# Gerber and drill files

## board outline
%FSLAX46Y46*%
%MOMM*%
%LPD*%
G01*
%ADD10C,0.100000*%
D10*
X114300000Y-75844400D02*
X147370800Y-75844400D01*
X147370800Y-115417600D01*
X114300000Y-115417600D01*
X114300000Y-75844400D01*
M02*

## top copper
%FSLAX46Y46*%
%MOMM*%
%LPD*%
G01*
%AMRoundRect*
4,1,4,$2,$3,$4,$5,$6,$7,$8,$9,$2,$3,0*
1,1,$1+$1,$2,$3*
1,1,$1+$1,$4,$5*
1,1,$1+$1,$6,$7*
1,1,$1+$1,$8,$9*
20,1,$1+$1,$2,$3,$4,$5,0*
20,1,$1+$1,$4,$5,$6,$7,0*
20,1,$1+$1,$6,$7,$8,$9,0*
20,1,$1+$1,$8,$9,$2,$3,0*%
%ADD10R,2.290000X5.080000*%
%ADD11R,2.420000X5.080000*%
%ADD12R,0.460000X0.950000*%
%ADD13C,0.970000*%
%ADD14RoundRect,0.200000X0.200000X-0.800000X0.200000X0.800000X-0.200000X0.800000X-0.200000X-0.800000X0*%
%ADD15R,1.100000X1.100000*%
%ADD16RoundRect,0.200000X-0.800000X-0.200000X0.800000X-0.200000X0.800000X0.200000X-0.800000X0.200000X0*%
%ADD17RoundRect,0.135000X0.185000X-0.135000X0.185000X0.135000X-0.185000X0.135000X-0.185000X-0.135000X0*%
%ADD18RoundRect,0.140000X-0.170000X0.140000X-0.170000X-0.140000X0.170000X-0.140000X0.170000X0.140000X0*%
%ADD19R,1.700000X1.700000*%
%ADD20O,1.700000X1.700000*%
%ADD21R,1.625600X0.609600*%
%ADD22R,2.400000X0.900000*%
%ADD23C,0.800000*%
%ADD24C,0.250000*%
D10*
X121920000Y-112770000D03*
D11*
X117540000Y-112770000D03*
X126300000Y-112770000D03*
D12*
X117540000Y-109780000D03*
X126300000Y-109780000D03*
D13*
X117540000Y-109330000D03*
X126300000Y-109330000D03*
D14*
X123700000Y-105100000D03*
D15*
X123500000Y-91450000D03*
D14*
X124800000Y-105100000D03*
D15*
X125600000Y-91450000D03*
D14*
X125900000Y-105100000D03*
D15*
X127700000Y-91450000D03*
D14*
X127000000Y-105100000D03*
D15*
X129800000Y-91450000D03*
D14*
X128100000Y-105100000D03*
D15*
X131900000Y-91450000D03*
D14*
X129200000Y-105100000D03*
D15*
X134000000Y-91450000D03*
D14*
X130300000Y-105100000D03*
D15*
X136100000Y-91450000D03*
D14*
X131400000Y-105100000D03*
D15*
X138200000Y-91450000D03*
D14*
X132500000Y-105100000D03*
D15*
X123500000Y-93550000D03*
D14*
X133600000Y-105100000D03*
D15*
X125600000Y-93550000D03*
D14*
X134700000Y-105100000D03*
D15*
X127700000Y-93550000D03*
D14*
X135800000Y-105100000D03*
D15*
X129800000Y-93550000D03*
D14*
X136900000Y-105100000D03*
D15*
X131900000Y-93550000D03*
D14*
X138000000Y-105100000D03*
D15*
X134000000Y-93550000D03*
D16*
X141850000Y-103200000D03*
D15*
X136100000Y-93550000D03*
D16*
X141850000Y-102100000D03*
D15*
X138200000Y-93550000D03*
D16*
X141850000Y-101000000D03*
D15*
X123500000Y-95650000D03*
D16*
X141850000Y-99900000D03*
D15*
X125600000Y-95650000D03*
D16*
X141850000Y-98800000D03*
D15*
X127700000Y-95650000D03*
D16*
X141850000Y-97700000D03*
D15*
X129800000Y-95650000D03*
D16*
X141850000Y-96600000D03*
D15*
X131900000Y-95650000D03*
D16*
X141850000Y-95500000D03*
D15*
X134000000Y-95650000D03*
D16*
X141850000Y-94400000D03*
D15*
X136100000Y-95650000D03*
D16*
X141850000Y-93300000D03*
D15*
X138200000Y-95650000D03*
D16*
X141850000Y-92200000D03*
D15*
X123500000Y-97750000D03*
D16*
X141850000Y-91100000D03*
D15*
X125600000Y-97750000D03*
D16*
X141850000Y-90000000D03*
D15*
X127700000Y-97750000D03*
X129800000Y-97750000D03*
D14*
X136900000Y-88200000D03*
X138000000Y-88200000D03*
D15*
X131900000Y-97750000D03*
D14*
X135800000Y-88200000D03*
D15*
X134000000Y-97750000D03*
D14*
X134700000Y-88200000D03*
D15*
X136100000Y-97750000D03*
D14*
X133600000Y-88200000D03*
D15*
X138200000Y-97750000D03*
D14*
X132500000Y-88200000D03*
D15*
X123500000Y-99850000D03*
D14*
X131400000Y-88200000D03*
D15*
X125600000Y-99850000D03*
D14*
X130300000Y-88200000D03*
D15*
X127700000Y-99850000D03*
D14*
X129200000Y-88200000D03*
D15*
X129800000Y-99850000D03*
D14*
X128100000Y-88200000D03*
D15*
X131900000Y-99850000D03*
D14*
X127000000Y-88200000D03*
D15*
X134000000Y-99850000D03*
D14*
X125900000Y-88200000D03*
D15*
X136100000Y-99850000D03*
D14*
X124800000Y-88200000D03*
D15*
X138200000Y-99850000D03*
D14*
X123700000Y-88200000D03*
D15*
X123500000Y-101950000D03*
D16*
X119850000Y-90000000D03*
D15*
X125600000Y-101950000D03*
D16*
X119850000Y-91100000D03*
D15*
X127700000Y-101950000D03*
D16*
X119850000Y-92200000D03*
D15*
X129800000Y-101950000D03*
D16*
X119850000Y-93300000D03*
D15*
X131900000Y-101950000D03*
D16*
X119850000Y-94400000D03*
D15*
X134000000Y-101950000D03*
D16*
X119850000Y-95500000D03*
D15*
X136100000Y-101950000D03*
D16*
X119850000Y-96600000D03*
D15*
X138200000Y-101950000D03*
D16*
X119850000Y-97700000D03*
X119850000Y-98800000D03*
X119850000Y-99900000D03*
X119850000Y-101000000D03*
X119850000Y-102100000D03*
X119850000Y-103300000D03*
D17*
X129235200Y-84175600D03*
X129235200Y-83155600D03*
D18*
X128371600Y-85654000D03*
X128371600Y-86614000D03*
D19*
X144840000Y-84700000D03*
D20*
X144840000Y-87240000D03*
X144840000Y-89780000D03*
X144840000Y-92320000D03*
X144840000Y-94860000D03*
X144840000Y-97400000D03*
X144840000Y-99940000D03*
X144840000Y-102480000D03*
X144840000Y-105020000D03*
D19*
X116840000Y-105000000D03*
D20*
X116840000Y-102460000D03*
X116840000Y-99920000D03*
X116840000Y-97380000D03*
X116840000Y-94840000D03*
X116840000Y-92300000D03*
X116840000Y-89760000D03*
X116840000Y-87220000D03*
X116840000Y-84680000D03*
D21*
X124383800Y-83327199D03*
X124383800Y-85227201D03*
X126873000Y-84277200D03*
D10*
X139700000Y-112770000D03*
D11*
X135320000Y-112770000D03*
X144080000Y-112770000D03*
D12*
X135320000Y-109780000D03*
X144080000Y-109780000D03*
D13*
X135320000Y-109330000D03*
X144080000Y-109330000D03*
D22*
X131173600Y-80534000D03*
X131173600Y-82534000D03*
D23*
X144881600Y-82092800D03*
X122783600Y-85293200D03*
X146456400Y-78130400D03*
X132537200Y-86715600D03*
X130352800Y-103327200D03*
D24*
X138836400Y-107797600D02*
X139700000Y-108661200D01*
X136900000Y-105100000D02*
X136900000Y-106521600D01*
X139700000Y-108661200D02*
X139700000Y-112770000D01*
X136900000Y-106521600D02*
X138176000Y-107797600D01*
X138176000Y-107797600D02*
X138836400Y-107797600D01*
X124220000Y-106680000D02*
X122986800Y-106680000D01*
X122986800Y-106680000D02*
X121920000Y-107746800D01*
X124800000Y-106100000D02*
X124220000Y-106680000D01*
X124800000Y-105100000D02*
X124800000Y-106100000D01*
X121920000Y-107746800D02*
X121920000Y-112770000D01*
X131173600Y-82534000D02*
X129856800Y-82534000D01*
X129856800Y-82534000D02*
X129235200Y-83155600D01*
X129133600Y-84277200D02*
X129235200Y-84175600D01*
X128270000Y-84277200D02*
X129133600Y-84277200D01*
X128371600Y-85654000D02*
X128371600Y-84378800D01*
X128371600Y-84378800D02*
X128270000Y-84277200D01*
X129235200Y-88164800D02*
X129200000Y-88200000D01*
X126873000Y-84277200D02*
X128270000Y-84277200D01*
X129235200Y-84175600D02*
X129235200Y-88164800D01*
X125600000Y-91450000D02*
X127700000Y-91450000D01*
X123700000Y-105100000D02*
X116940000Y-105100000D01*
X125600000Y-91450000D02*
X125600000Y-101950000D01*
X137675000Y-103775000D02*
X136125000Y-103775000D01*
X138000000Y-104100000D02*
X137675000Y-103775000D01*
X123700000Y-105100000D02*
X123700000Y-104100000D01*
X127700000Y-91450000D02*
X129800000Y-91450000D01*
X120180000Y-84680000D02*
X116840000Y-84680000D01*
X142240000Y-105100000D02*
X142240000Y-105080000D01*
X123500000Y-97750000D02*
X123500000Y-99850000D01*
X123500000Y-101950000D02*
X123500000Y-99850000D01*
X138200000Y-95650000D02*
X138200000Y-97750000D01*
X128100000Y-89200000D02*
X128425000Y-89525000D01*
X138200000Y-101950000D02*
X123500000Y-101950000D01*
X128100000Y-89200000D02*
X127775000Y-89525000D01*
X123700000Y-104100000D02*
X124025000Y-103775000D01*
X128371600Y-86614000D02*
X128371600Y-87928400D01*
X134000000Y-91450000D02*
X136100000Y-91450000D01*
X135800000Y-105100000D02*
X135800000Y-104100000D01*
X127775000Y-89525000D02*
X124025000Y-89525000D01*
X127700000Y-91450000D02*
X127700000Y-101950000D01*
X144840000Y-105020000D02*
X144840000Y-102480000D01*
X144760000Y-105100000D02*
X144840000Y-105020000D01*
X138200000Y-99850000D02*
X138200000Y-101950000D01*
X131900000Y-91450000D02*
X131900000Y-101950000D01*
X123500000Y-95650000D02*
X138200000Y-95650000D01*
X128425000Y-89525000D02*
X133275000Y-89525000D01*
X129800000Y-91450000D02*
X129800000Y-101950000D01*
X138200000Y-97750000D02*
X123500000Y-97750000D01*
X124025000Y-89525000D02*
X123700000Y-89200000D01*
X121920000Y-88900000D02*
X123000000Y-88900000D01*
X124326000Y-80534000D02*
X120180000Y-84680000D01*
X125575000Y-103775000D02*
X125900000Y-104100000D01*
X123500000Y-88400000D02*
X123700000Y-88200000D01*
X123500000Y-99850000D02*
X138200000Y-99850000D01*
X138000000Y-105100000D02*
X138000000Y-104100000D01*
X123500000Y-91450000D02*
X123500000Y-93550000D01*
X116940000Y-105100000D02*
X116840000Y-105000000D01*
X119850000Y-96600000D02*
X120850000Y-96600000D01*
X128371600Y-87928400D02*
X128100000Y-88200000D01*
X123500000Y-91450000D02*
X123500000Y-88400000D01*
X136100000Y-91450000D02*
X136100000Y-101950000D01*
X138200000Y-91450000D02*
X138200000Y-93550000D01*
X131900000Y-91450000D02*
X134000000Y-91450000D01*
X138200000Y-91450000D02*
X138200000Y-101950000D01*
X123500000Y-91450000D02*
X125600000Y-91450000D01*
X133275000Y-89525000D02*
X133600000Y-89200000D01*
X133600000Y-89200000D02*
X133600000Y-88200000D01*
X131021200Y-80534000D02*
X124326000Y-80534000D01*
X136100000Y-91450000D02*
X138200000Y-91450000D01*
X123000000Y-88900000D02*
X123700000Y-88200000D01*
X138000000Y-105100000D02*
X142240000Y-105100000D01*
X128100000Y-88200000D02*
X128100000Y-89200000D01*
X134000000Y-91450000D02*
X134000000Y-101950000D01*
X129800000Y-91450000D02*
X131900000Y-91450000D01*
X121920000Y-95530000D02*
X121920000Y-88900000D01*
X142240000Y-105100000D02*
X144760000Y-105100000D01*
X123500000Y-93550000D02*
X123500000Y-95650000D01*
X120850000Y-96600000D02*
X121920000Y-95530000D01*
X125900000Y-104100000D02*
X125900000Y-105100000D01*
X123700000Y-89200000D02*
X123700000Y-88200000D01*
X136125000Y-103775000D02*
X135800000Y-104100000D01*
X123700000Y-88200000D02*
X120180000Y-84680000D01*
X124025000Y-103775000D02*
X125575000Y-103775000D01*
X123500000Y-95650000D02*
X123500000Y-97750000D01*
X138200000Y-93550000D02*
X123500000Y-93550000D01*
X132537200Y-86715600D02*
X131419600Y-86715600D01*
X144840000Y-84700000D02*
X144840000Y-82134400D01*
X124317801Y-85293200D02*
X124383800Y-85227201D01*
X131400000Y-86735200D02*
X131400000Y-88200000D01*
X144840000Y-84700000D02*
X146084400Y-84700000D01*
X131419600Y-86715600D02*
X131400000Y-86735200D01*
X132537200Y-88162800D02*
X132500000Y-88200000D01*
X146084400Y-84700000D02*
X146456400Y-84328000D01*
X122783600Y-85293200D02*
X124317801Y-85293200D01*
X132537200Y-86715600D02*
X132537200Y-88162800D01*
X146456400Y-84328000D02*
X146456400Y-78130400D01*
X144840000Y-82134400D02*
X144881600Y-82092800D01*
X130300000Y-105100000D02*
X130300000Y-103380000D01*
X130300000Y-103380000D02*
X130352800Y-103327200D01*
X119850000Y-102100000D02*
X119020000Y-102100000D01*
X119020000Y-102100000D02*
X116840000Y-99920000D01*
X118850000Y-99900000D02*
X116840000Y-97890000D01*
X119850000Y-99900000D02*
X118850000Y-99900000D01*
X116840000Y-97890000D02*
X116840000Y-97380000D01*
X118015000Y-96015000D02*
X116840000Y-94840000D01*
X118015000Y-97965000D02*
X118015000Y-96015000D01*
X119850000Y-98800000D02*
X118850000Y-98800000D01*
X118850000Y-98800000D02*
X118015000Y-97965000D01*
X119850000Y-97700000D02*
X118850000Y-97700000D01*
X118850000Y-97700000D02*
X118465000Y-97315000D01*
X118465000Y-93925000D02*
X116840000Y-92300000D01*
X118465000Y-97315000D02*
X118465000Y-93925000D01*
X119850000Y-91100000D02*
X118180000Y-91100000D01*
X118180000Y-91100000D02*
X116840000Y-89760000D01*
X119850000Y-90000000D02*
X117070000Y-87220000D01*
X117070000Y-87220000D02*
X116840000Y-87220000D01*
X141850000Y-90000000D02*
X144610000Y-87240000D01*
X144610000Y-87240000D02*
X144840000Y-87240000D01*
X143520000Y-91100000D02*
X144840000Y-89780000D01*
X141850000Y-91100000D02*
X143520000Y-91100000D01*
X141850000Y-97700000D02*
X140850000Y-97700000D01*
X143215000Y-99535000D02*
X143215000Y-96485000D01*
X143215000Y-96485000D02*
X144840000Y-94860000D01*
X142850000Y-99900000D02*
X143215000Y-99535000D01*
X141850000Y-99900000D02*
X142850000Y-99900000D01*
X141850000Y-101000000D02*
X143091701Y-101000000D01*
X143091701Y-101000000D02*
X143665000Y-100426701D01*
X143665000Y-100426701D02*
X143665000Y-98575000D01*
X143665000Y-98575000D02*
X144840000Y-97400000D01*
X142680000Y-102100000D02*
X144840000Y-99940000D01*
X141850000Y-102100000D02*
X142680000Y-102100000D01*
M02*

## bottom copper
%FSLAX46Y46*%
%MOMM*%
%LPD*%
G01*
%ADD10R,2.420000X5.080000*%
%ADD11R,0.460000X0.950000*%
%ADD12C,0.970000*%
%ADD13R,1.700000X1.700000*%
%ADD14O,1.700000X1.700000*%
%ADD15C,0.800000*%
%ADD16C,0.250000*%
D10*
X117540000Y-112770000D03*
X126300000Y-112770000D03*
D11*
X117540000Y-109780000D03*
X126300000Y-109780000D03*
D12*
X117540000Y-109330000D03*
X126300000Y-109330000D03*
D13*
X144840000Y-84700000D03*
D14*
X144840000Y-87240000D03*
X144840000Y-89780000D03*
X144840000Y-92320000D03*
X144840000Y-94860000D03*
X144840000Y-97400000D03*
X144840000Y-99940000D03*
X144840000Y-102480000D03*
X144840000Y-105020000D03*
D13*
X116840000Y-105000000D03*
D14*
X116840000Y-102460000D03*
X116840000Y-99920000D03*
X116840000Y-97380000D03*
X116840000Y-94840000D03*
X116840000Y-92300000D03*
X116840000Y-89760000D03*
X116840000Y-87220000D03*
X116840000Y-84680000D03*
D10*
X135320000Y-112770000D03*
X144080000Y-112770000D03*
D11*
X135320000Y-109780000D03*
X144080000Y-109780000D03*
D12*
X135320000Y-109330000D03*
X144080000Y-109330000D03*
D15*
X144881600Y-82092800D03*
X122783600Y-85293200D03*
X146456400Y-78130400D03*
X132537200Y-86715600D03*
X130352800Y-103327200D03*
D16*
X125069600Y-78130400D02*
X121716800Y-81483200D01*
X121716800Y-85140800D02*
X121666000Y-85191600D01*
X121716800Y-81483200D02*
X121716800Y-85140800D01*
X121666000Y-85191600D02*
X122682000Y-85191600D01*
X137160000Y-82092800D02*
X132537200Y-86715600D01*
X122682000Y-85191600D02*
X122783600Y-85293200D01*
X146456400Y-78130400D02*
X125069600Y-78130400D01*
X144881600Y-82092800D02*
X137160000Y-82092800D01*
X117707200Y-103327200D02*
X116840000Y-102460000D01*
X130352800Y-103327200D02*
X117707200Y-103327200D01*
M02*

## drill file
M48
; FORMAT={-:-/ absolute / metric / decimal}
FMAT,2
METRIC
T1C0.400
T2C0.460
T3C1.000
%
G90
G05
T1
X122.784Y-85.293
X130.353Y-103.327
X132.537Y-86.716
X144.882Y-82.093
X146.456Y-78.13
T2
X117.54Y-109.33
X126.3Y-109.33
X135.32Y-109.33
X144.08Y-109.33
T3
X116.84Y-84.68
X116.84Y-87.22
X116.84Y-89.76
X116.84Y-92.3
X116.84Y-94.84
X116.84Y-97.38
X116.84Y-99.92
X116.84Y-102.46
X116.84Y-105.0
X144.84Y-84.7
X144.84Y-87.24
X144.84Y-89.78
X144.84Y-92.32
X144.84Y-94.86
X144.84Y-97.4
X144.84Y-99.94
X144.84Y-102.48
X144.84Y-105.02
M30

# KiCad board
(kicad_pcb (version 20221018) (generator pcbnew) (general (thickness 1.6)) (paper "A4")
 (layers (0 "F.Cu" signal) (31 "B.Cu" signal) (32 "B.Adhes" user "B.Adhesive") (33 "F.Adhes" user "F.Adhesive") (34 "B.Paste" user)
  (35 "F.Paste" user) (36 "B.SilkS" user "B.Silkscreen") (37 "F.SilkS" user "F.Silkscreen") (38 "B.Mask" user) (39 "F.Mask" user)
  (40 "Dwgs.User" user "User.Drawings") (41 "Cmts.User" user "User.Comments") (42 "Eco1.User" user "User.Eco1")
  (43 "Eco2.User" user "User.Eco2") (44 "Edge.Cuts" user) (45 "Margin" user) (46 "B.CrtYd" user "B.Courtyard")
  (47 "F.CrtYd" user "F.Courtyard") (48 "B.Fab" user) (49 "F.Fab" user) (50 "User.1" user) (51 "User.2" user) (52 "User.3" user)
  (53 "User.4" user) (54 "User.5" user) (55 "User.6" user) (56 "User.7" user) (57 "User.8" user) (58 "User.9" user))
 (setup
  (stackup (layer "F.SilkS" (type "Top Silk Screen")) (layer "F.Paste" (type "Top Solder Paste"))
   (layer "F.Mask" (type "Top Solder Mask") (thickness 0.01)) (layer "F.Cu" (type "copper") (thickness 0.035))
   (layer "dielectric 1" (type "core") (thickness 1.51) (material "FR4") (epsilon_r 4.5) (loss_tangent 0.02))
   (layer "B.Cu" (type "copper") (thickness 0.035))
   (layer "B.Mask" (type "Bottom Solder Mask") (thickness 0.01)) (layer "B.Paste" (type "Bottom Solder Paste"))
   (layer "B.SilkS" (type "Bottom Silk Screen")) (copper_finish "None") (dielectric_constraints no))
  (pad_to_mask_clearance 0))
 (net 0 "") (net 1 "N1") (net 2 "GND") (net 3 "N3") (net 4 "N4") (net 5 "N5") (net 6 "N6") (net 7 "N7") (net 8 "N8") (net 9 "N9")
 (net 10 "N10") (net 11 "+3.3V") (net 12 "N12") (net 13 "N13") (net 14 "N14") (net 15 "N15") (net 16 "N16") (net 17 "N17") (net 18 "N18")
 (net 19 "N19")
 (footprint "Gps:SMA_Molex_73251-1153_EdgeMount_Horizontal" (layer "F.Cu") (at 121.92 111.05 90)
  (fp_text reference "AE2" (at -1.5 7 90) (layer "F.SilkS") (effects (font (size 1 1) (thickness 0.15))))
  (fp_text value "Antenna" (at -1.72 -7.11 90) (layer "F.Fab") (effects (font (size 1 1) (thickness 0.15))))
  (pad "1" smd rect (at -1.72 0 90) (size 5.08 2.29) (layers "F.Cu" "F.Paste" "F.Mask") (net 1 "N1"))
  (pad "2" smd rect (at -1.72 -4.38 90) (size 5.08 2.42) (layers "F.Cu" "F.Paste" "F.Mask"))
  (pad "2" smd rect (at -1.72 -4.38 90) (size 5.08 2.42) (layers "B.Cu" "B.Paste" "B.Mask"))
  (pad "2" smd rect (at -1.72 4.38 90) (size 5.08 2.42) (layers "F.Cu" "F.Paste" "F.Mask"))
  (pad "2" smd rect (at -1.72 4.38 90) (size 5.08 2.42) (layers "B.Cu" "B.Paste" "B.Mask"))
  (pad "2" smd rect (at 1.27 -4.38 90) (size 0.95 0.46) (layers "F.Cu"))
  (pad "2" smd rect (at 1.27 -4.38 90) (size 0.95 0.46) (layers "B.Cu"))
  (pad "2" smd rect (at 1.27 4.38 90) (size 0.95 0.46) (layers "F.Cu"))
  (pad "2" smd rect (at 1.27 4.38 90) (size 0.95 0.46) (layers "B.Cu"))
  (pad "2" thru_hole circle (at 1.72 -4.38 90) (size 0.97 0.97) (drill 0.46) (layers "*.Cu"))
  (pad "2" thru_hole circle (at 1.72 4.38 90) (size 0.97 0.97) (drill 0.46) (layers "*.Cu")))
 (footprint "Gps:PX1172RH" (layer "F.Cu") (at 119.85 90)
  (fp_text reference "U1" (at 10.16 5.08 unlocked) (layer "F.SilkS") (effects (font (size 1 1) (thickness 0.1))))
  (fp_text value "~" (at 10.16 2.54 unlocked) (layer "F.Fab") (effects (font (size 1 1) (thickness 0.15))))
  (pad "1" smd roundrect (at 3.85 15.1 90) (size 2 0.8) (layers "F.Cu" "F.Paste" "F.Mask") (roundrect_rratio 0.25) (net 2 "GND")
   (thermal_bridge_angle 45))
  (pad "1$" smd rect (at 3.65 1.45) (size 1.1 1.1) (layers "F.Cu" "F.Paste" "F.Mask") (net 2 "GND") (thermal_bridge_angle 45))
  (pad "2" smd roundrect (at 4.95 15.1 90) (size 2 0.8) (layers "F.Cu" "F.Paste" "F.Mask") (roundrect_rratio 0.25) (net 1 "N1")
   (thermal_bridge_angle 45))
  (pad "2$" smd rect (at 5.75 1.45) (size 1.1 1.1) (layers "F.Cu" "F.Paste" "F.Mask") (thermal_bridge_angle 45))
  (pad "3" smd roundrect (at 6.05 15.1 90) (size 2 0.8) (layers "F.Cu" "F.Paste" "F.Mask") (roundrect_rratio 0.25) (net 2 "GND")
   (thermal_bridge_angle 45))
  (pad "3$" smd rect (at 7.85 1.45) (size 1.1 1.1) (layers "F.Cu" "F.Paste" "F.Mask") (thermal_bridge_angle 45))
  (pad "4" smd roundrect (at 7.15 15.1 90) (size 2 0.8) (layers "F.Cu" "F.Paste" "F.Mask") (roundrect_rratio 0.25) (thermal_bridge_angle 45))
  (pad "4$" smd rect (at 9.95 1.45) (size 1.1 1.1) (layers "F.Cu" "F.Paste" "F.Mask") (thermal_bridge_angle 45))
  (pad "5" smd roundrect (at 8.25 15.1 90) (size 2 0.8) (layers "F.Cu" "F.Paste" "F.Mask") (roundrect_rratio 0.25) (thermal_bridge_angle 45))
  (pad "5$" smd rect (at 12.05 1.45) (size 1.1 1.1) (layers "F.Cu" "F.Paste" "F.Mask") (thermal_bridge_angle 45))
  (pad "6" smd roundrect (at 9.35 15.1 90) (size 2 0.8) (layers "F.Cu" "F.Paste" "F.Mask") (roundrect_rratio 0.25) (thermal_bridge_angle 45))
  (pad "6$" smd rect (at 14.15 1.45) (size 1.1 1.1) (layers "F.Cu" "F.Paste" "F.Mask") (thermal_bridge_angle 45))
  (pad "7" smd roundrect (at 10.45 15.1 90) (size 2 0.8) (layers "F.Cu" "F.Paste" "F.Mask") (roundrect_rratio 0.25) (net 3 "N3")
   (thermal_bridge_angle 45))
  (pad "7$" smd rect (at 16.25 1.45) (size 1.1 1.1) (layers "F.Cu" "F.Paste" "F.Mask") (thermal_bridge_angle 45))
  (pad "8" smd roundrect (at 11.55 15.1 90) (size 2 0.8) (layers "F.Cu" "F.Paste" "F.Mask") (roundrect_rratio 0.25)
   (thermal_bridge_angle 45))
  (pad "8$" smd rect (at 18.35 1.45) (size 1.1 1.1) (layers "F.Cu" "F.Paste" "F.Mask") (thermal_bridge_angle 45))
  (pad "9" smd roundrect (at 12.65 15.1 90) (size 2 0.8) (layers "F.Cu" "F.Paste" "F.Mask") (roundrect_rratio 0.25)
   (thermal_bridge_angle 45))
  (pad "9$" smd rect (at 3.65 3.55) (size 1.1 1.1) (layers "F.Cu" "F.Paste" "F.Mask") (thermal_bridge_angle 45))
  (pad "10" smd roundrect (at 13.75 15.1 90) (size 2 0.8) (layers "F.Cu" "F.Paste" "F.Mask") (roundrect_rratio 0.25)
   (thermal_bridge_angle 45))
  (pad "10$" smd rect (at 5.75 3.55) (size 1.1 1.1) (layers "F.Cu" "F.Paste" "F.Mask") (thermal_bridge_angle 45))
  (pad "11" smd roundrect (at 14.85 15.1 90) (size 2 0.8) (layers "F.Cu" "F.Paste" "F.Mask") (roundrect_rratio 0.25)
   (thermal_bridge_angle 45))
  (pad "11$" smd rect (at 7.85 3.55) (size 1.1 1.1) (layers "F.Cu" "F.Paste" "F.Mask") (thermal_bridge_angle 45))
  (pad "12" smd roundrect (at 15.95 15.1 90) (size 2 0.8) (layers "F.Cu" "F.Paste" "F.Mask") (roundrect_rratio 0.25) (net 2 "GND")
   (thermal_bridge_angle 45))
  (pad "12$" smd rect (at 9.95 3.55) (size 1.1 1.1) (layers "F.Cu" "F.Paste" "F.Mask") (thermal_bridge_angle 45))
  (pad "13" smd roundrect (at 17.05 15.1 90) (size 2 0.8) (layers "F.Cu" "F.Paste" "F.Mask") (roundrect_rratio 0.25) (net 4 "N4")
   (thermal_bridge_angle 45))
  (pad "13$" smd rect (at 12.05 3.55) (size 1.1 1.1) (layers "F.Cu" "F.Paste" "F.Mask") (thermal_bridge_angle 45))
  (pad "14" smd roundrect (at 18.15 15.1 90) (size 2 0.8) (layers "F.Cu" "F.Paste" "F.Mask") (roundrect_rratio 0.25) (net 2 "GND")
   (thermal_bridge_angle 45))
  (pad "14$" smd rect (at 14.15 3.55) (size 1.1 1.1) (layers "F.Cu" "F.Paste" "F.Mask") (thermal_bridge_angle 45))
  (pad "15" smd roundrect (at 22 13.2) (size 2 0.8) (layers "F.Cu" "F.Paste" "F.Mask") (roundrect_rratio 0.25) (thermal_bridge_angle 45))
  (pad "15$" smd rect (at 16.25 3.55) (size 1.1 1.1) (layers "F.Cu" "F.Paste" "F.Mask") (thermal_bridge_angle 45))
  (pad "16" smd roundrect (at 22 12.1) (size 2 0.8) (layers "F.Cu" "F.Paste" "F.Mask") (roundrect_rratio 0.25) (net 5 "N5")
   (thermal_bridge_angle 45))
  (pad "16$" smd rect (at 18.35 3.55) (size 1.1 1.1) (layers "F.Cu" "F.Paste" "F.Mask") (thermal_bridge_angle 45))
  (pad "17" smd roundrect (at 22 11) (size 2 0.8) (layers "F.Cu" "F.Paste" "F.Mask") (roundrect_rratio 0.25) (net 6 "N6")
   (thermal_bridge_angle 45))
  (pad "17$" smd rect (at 3.65 5.65) (size 1.1 1.1) (layers "F.Cu" "F.Paste" "F.Mask") (thermal_bridge_angle 45))
  (pad "18" smd roundrect (at 22 9.9) (size 2 0.8) (layers "F.Cu" "F.Paste" "F.Mask") (roundrect_rratio 0.25) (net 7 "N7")
   (thermal_bridge_angle 45))
  (pad "18$" smd rect (at 5.75 5.65) (size 1.1 1.1) (layers "F.Cu" "F.Paste" "F.Mask") (thermal_bridge_angle 45))
  (pad "19" smd roundrect (at 22 8.8) (size 2 0.8) (layers "F.Cu" "F.Paste" "F.Mask") (roundrect_rratio 0.25) (thermal_bridge_angle 45))
  (pad "19$" smd rect (at 7.85 5.65) (size 1.1 1.1) (layers "F.Cu" "F.Paste" "F.Mask") (thermal_bridge_angle 45))
  (pad "20" smd roundrect (at 22 7.7) (size 2 0.8) (layers "F.Cu" "F.Paste" "F.Mask") (roundrect_rratio 0.25) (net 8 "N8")
   (thermal_bridge_angle 45))
  (pad "20$" smd rect (at 9.95 5.65) (size 1.1 1.1) (layers "F.Cu" "F.Paste" "F.Mask") (thermal_bridge_angle 45))
  (pad "21" smd roundrect (at 22 6.6) (size 2 0.8) (layers "F.Cu" "F.Paste" "F.Mask") (roundrect_rratio 0.25) (thermal_bridge_angle 45))
  (pad "21$" smd rect (at 12.05 5.65) (size 1.1 1.1) (layers "F.Cu" "F.Paste" "F.Mask") (thermal_bridge_angle 45))
  (pad "22" smd roundrect (at 22 5.5) (size 2 0.8) (layers "F.Cu" "F.Paste" "F.Mask") (roundrect_rratio 0.25) (thermal_bridge_angle 45))
  (pad "22$" smd rect (at 14.15 5.65) (size 1.1 1.1) (layers "F.Cu" "F.Paste" "F.Mask") (thermal_bridge_angle 45))
  (pad "23" smd roundrect (at 22 4.4) (size 2 0.8) (layers "F.Cu" "F.Paste" "F.Mask") (roundrect_rratio 0.25) (thermal_bridge_angle 45))
  (pad "23$" smd rect (at 16.25 5.65) (size 1.1 1.1) (layers "F.Cu" "F.Paste" "F.Mask") (thermal_bridge_angle 45))
  (pad "24" smd roundrect (at 22 3.3) (size 2 0.8) (layers "F.Cu" "F.Paste" "F.Mask") (roundrect_rratio 0.25) (thermal_bridge_angle 45))
  (pad "24$" smd rect (at 18.35 5.65) (size 1.1 1.1) (layers "F.Cu" "F.Paste" "F.Mask") (thermal_bridge_angle 45))
  (pad "25" smd roundrect (at 22 2.2) (size 2 0.8) (layers "F.Cu" "F.Mask") (roundrect_rratio 0.25) (thermal_bridge_angle 45))
  (pad "25$" smd rect (at 3.65 7.75) (size 1.1 1.1) (layers "F.Cu" "F.Paste" "F.Mask") (thermal_bridge_angle 45))
  (pad "26" smd roundrect (at 22 1.1) (size 2 0.8) (layers "F.Cu" "F.Paste" "F.Mask") (roundrect_rratio 0.25) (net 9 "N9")
   (thermal_bridge_angle 45))
  (pad "26$" smd rect (at 5.75 7.75) (size 1.1 1.1) (layers "F.Cu" "F.Paste" "F.Mask") (thermal_bridge_angle 45))
  (pad "27" smd roundrect (at 22 0) (size 2 0.8) (layers "F.Cu" "F.Paste" "F.Mask") (roundrect_rratio 0.25) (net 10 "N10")
   (thermal_bridge_angle 45))
  (pad "27$" smd rect (at 7.85 7.75) (size 1.1 1.1) (layers "F.Cu" "F.Paste" "F.Mask") (thermal_bridge_angle 45))
  (pad "28$" smd rect (at 9.95 7.75) (size 1.1 1.1) (layers "F.Cu" "F.Paste" "F.Mask") (thermal_bridge_angle 45))
  (pad "29" smd roundrect (at 17.05 -1.8 90) (size 2 0.8) (layers "F.Cu" "F.Paste" "F.Mask") (roundrect_rratio 0.25)
   (thermal_bridge_angle 45))
  (pad "29" smd roundrect (at 18.15 -1.8 90) (size 2 0.8) (layers "F.Cu" "F.Paste" "F.Mask") (roundrect_rratio 0.25)
   (thermal_bridge_angle 45))
  (pad "29$" smd rect (at 12.05 7.75) (size 1.1 1.1) (layers "F.Cu" "F.Paste" "F.Mask") (thermal_bridge_angle 45))
  (pad "30" smd roundrect (at 15.95 -1.8 90) (size 2 0.8) (layers "F.Cu" "F.Paste" "F.Mask") (roundrect_rratio 0.25)
   (thermal_bridge_angle 45))
  (pad "30$" smd rect (at 14.15 7.75) (size 1.1 1.1) (layers "F.Cu" "F.Paste" "F.Mask") (thermal_bridge_angle 45))
  (pad "31" smd roundrect (at 14.85 -1.8 90) (size 2 0.8) (layers "F.Cu" "F.Paste" "F.Mask") (roundrect_rratio 0.25)
   (thermal_bridge_angle 45))
  (pad "31$" smd rect (at 16.25 7.75) (size 1.1 1.1) (layers "F.Cu" "F.Paste" "F.Mask") (thermal_bridge_angle 45))
  (pad "32" smd roundrect (at 13.75 -1.8 90) (size 2 0.8) (layers "F.Cu" "F.Paste" "F.Mask") (roundrect_rratio 0.25) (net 2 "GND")
   (thermal_bridge_angle 45))
  (pad "32$" smd rect (at 18.35 7.75) (size 1.1 1.1) (layers "F.Cu" "F.Paste" "F.Mask") (thermal_bridge_angle 45))
  (pad "33" smd roundrect (at 12.65 -1.8 90) (size 2 0.8) (layers "F.Cu" "F.Paste" "F.Mask") (roundrect_rratio 0.25) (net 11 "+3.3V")
   (thermal_bridge_angle 45))
  (pad "33$" smd rect (at 3.65 9.85) (size 1.1 1.1) (layers "F.Cu" "F.Paste" "F.Mask") (thermal_bridge_angle 45))
  (pad "34" smd roundrect (at 11.55 -1.8 90) (size 2 0.8) (layers "F.Cu" "F.Paste" "F.Mask") (roundrect_rratio 0.25) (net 11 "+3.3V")
   (thermal_bridge_angle 45))
  (pad "34$" smd rect (at 5.75 9.85) (size 1.1 1.1) (layers "F.Cu" "F.Paste" "F.Mask") (thermal_bridge_angle 45))
  (pad "35" smd roundrect (at 10.45 -1.8 90) (size 2 0.8) (layers "F.Cu" "F.Paste" "F.Mask") (roundrect_rratio 0.25)
   (thermal_bridge_angle 45))
  (pad "35$" smd rect (at 7.85 9.85) (size 1.1 1.1) (layers "F.Cu" "F.Paste" "F.Mask") (thermal_bridge_angle 45))
  (pad "36" smd roundrect (at 9.35 -1.8 90) (size 2 0.8) (layers "F.Cu" "F.Paste" "F.Mask") (roundrect_rratio 0.25) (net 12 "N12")
   (thermal_bridge_angle 45))
  (pad "36$" smd rect (at 9.95 9.85) (size 1.1 1.1) (layers "F.Cu" "F.Paste" "F.Mask") (thermal_bridge_angle 45))
  (pad "37" smd roundrect (at 8.25 -1.8 90) (size 2 0.8) (layers "F.Cu" "F.Paste" "F.Mask") (roundrect_rratio 0.25) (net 2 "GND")
   (thermal_bridge_angle 45))
  (pad "37$" smd rect (at 12.05 9.85) (size 1.1 1.1) (layers "F.Cu" "F.Paste" "F.Mask") (thermal_bridge_angle 45))
  (pad "38" smd roundrect (at 7.15 -1.8 90) (size 2 0.8) (layers "F.Cu" "F.Paste" "F.Mask") (roundrect_rratio 0.25)
   (thermal_bridge_angle 45))
  (pad "38$" smd rect (at 14.15 9.85) (size 1.1 1.1) (layers "F.Cu" "F.Paste" "F.Mask") (thermal_bridge_angle 45))
  (pad "39" smd roundrect (at 6.05 -1.8 90) (size 2 0.8) (layers "F.Cu" "F.Paste" "F.Mask") (roundrect_rratio 0.25)
   (thermal_bridge_angle 45))
  (pad "39$" smd rect (at 16.25 9.85) (size 1.1 1.1) (layers "F.Cu" "F.Paste" "F.Mask") (thermal_bridge_angle 45))
  (pad "40" smd roundrect (at 4.95 -1.8 90) (size 2 0.8) (layers "F.Cu" "F.Paste" "F.Mask") (roundrect_rratio 0.25)
   (thermal_bridge_angle 45))
  (pad "40$" smd rect (at 18.35 9.85) (size 1.1 1.1) (layers "F.Cu" "F.Paste" "F.Mask") (thermal_bridge_angle 45))
  (pad "41" smd roundrect (at 3.85 -1.8 90) (size 2 0.8) (layers "F.Cu" "F.Paste" "F.Mask") (roundrect_rratio 0.25) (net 2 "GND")
   (thermal_bridge_angle 45))
  (pad "41$" smd rect (at 3.65 11.95) (size 1.1 1.1) (layers "F.Cu" "F.Paste" "F.Mask") (thermal_bridge_angle 45))
  (pad "42" smd roundrect (at 0 0) (size 2 0.8) (layers "F.Cu" "F.Paste" "F.Mask") (roundrect_rratio 0.25) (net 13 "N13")
   (thermal_bridge_angle 45))
  (pad "42$" smd rect (at 5.75 11.95) (size 1.1 1.1) (layers "F.Cu" "F.Paste" "F.Mask") (thermal_bridge_angle 45))
  (pad "43" smd roundrect (at 0 1.1) (size 2 0.8) (layers "F.Cu" "F.Paste" "F.Mask") (roundrect_rratio 0.25) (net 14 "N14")
   (thermal_bridge_angle 45))
  (pad "43$" smd rect (at 7.85 11.95) (size 1.1 1.1) (layers "F.Cu" "F.Paste" "F.Mask") (thermal_bridge_angle 45))
  (pad "44" smd roundrect (at 0 2.2) (size 2 0.8) (layers "F.Cu" "F.Paste" "F.Mask") (roundrect_rratio 0.25) (thermal_bridge_angle 45))
  (pad "44$" smd rect (at 9.95 11.95) (size 1.1 1.1) (layers "F.Cu" "F.Paste" "F.Mask") (thermal_bridge_angle 45))
  (pad "45" smd roundrect (at 0 3.3) (size 2 0.8) (layers "F.Cu" "F.Paste" "F.Mask") (roundrect_rratio 0.25) (thermal_bridge_angle 45))
  (pad "45$" smd rect (at 12.05 11.95) (size 1.1 1.1) (layers "F.Cu" "F.Paste" "F.Mask") (thermal_bridge_angle 45))
  (pad "46" smd roundrect (at 0 4.4) (size 2 0.8) (layers "F.Cu" "F.Paste" "F.Mask") (roundrect_rratio 0.25) (thermal_bridge_angle 45))
  (pad "46$" smd rect (at 14.15 11.95) (size 1.1 1.1) (layers "F.Cu" "F.Paste" "F.Mask") (thermal_bridge_angle 45))
  (pad "47" smd roundrect (at 0 5.5) (size 2 0.8) (layers "F.Cu" "F.Paste" "F.Mask") (roundrect_rratio 0.25) (thermal_bridge_angle 45))
  (pad "47$" smd rect (at 16.25 11.95) (size 1.1 1.1) (layers "F.Cu" "F.Paste" "F.Mask") (thermal_bridge_angle 45))
  (pad "48" smd roundrect (at 0 6.6) (size 2 0.8) (layers "F.Cu" "F.Paste" "F.Mask") (roundrect_rratio 0.25) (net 2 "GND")
   (thermal_bridge_angle 45))
  (pad "48$" smd rect (at 18.35 11.95) (size 1.1 1.1) (layers "F.Cu" "F.Paste" "F.Mask") (thermal_bridge_angle 45))
  (pad "49" smd roundrect (at 0 7.7) (size 2 0.8) (layers "F.Cu" "F.Paste" "F.Mask") (roundrect_rratio 0.25) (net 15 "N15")
   (thermal_bridge_angle 45))
  (pad "50" smd roundrect (at 0 8.8) (size 2 0.8) (layers "F.Cu" "F.Paste" "F.Mask") (roundrect_rratio 0.25) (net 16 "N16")
   (thermal_bridge_angle 45))
  (pad "51" smd roundrect (at 0 9.9) (size 2 0.8) (layers "F.Cu" "F.Paste" "F.Mask") (roundrect_rratio 0.25) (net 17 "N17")
   (thermal_bridge_angle 45))
  (pad "52" smd roundrect (at 0 11) (size 2 0.8) (layers "F.Cu" "F.Paste" "F.Mask") (roundrect_rratio 0.25) (thermal_bridge_angle 45))
  (pad "53" smd roundrect (at 0 12.1) (size 2 0.8) (layers "F.Cu" "F.Paste" "F.Mask") (roundrect_rratio 0.25) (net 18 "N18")
   (thermal_bridge_angle 45))
  (pad "54" smd roundrect (at 0 13.3) (size 2 0.8) (layers "F.Cu" "F.Paste" "F.Mask") (roundrect_rratio 0.25) (thermal_bridge_angle 45)))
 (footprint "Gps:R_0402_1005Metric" (layer "F.Cu") (at 129.2352 83.6656 90)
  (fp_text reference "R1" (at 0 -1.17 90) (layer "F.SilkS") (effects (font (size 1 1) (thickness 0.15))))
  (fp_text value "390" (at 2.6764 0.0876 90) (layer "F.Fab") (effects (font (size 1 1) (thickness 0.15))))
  (pad "1" smd roundrect (at -0.51 0 90) (size 0.54 0.64) (layers "F.Cu" "F.Paste" "F.Mask") (roundrect_rratio 0.25) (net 12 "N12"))
  (pad "2" smd roundrect (at 0.51 0 90) (size 0.54 0.64) (layers "F.Cu" "F.Paste" "F.Mask") (roundrect_rratio 0.25) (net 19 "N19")))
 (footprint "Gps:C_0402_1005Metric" (layer "F.Cu") (at 128.3716 86.134 -90)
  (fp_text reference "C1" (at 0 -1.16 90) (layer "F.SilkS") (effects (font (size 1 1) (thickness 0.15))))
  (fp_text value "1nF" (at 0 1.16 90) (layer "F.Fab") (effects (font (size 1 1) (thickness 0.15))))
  (pad "1" smd roundrect (at -0.48 0 270) (size 0.56 0.62) (layers "F.Cu" "F.Paste" "F.Mask") (roundrect_rratio 0.25) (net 12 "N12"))
  (pad "2" smd roundrect (at 0.48 0 270) (size 0.56 0.62) (layers "F.Cu" "F.Paste" "F.Mask") (roundrect_rratio 0.25) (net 2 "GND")))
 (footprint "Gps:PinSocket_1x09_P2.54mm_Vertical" (layer "F.Cu") (at 144.84 84.7)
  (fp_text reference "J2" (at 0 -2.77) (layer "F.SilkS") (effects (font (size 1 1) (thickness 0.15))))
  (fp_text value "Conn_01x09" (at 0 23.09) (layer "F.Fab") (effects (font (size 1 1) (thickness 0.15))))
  (pad "1" thru_hole rect (at 0 0) (size 1.7 1.7) (drill 1) (layers "*.Cu" "*.Mask") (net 11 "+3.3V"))
  (pad "2" thru_hole oval (at 0 2.54) (size 1.7 1.7) (drill 1) (layers "*.Cu" "*.Mask") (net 10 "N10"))
  (pad "3" thru_hole oval (at 0 5.08) (size 1.7 1.7) (drill 1) (layers "*.Cu" "*.Mask") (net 9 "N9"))
  (pad "4" thru_hole oval (at 0 7.62) (size 1.7 1.7) (drill 1) (layers "*.Cu" "*.Mask") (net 8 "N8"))
  (pad "5" thru_hole oval (at 0 10.16) (size 1.7 1.7) (drill 1) (layers "*.Cu" "*.Mask") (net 7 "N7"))
  (pad "6" thru_hole oval (at 0 12.7) (size 1.7 1.7) (drill 1) (layers "*.Cu" "*.Mask") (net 6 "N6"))
  (pad "7" thru_hole oval (at 0 15.24) (size 1.7 1.7) (drill 1) (layers "*.Cu" "*.Mask") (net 5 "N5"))
  (pad "8" thru_hole oval (at 0 17.78) (size 1.7 1.7) (drill 1) (layers "*.Cu" "*.Mask") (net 2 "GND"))
  (pad "9" thru_hole oval (at 0 20.32) (size 1.7 1.7) (drill 1) (layers "*.Cu" "*.Mask") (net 2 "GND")))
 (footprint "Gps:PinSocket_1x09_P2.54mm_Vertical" (layer "F.Cu") (at 116.84 105 180)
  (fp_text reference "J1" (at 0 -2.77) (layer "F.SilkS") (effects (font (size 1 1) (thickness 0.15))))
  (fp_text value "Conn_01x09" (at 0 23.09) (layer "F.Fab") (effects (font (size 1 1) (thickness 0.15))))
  (pad "1" thru_hole rect (at 0 0 180) (size 1.7 1.7) (drill 1) (layers "*.Cu" "*.Mask") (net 2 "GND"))
  (pad "2" thru_hole oval (at 0 2.54 180) (size 1.7 1.7) (drill 1) (layers "*.Cu" "*.Mask") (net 3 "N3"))
  (pad "3" thru_hole oval (at 0 5.08 180) (size 1.7 1.7) (drill 1) (layers "*.Cu" "*.Mask") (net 18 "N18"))
  (pad "4" thru_hole oval (at 0 7.62 180) (size 1.7 1.7) (drill 1) (layers "*.Cu" "*.Mask") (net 17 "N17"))
  (pad "5" thru_hole oval (at 0 10.16 180) (size 1.7 1.7) (drill 1) (layers "*.Cu" "*.Mask") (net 16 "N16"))
  (pad "6" thru_hole oval (at 0 12.7 180) (size 1.7 1.7) (drill 1) (layers "*.Cu" "*.Mask") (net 15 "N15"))
  (pad "7" thru_hole oval (at 0 15.24 180) (size 1.7 1.7) (drill 1) (layers "*.Cu" "*.Mask") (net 14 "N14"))
  (pad "8" thru_hole oval (at 0 17.78 180) (size 1.7 1.7) (drill 1) (layers "*.Cu" "*.Mask") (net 13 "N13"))
  (pad "9" thru_hole oval (at 0 20.32 180) (size 1.7 1.7) (drill 1) (layers "*.Cu" "*.Mask") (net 2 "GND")))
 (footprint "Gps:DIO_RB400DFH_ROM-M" (layer "F.Cu") (at 125.6284 84.2772 -90)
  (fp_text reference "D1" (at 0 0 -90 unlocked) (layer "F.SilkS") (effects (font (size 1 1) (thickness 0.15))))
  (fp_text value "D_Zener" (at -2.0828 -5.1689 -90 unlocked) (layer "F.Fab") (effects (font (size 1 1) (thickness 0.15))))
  (pad "1" smd rect (at -0.950001 1.2446 270) (size 0.6096 1.6256) (layers "F.Cu" "F.Paste" "F.Mask"))
  (pad "2" smd rect (at 0.950001 1.2446 270) (size 0.6096 1.6256) (layers "F.Cu" "F.Paste" "F.Mask") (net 11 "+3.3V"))
  (pad "3" smd rect (at 0 -1.2446 270) (size 0.6096 1.6256) (layers "F.Cu" "F.Paste" "F.Mask") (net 12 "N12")))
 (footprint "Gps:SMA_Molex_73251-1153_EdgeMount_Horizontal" (layer "F.Cu") (at 139.7 111.05 90)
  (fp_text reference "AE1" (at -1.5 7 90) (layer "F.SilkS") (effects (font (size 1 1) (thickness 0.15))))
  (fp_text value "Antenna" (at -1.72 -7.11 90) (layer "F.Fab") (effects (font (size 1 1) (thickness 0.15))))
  (pad "1" smd rect (at -1.72 0 90) (size 5.08 2.29) (layers "F.Cu" "F.Paste" "F.Mask") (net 4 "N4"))
  (pad "2" smd rect (at -1.72 -4.38 90) (size 5.08 2.42) (layers "F.Cu" "F.Paste" "F.Mask"))
  (pad "2" smd rect (at -1.72 -4.38 90) (size 5.08 2.42) (layers "B.Cu" "B.Paste" "B.Mask"))
  (pad "2" smd rect (at -1.72 4.38 90) (size 5.08 2.42) (layers "F.Cu" "F.Paste" "F.Mask"))
  (pad "2" smd rect (at -1.72 4.38 90) (size 5.08 2.42) (layers "B.Cu" "B.Paste" "B.Mask"))
  (pad "2" smd rect (at 1.27 -4.38 90) (size 0.95 0.46) (layers "F.Cu"))
  (pad "2" smd rect (at 1.27 -4.38 90) (size 0.95 0.46) (layers "B.Cu"))
  (pad "2" smd rect (at 1.27 4.38 90) (size 0.95 0.46) (layers "F.Cu"))
  (pad "2" smd rect (at 1.27 4.38 90) (size 0.95 0.46) (layers "B.Cu"))
  (pad "2" thru_hole circle (at 1.72 -4.38 90) (size 0.97 0.97) (drill 0.46) (layers "*.Cu"))
  (pad "2" thru_hole circle (at 1.72 4.38 90) (size 0.97 0.97) (drill 0.46) (layers "*.Cu")))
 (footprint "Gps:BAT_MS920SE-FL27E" (layer "F.Cu") (at 138.0236 81.534 90)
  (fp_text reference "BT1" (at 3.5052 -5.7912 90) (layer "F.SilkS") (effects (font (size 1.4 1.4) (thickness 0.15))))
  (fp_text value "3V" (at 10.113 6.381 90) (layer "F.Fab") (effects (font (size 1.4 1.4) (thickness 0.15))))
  (pad "N" smd rect (at 1 -6.85 180) (size 2.4 0.9) (layers "F.Cu" "F.Paste" "F.Mask") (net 2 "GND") (solder_mask_margin 0.102))
  (pad "P" smd rect (at -1 -6.85 180) (size 2.4 0.9) (layers "F.Cu" "F.Paste" "F.Mask") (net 19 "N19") (solder_mask_margin 0.102)))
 (gr_rect (start 114.3 75.8444) (end 147.3708 115.4176) (stroke (width 0.1) (type default)) (fill none) (layer "Edge.Cuts"))
 (segment (start 138.8364 107.7976) (end 139.7 108.6612) (width 0.25) (layer "F.Cu") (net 4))
 (segment (start 136.9 105.1) (end 136.9 106.5216) (width 0.25) (layer "F.Cu") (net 4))
 (segment (start 139.7 108.6612) (end 139.7 112.77) (width 0.25) (layer "F.Cu") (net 4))
 (segment (start 136.9 106.5216) (end 138.176 107.7976) (width 0.25) (layer "F.Cu") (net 4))
 (segment (start 138.176 107.7976) (end 138.8364 107.7976) (width 0.25) (layer "F.Cu") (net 4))
 (segment (start 124.22 106.68) (end 122.9868 106.68) (width 0.25) (layer "F.Cu") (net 1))
 (segment (start 122.9868 106.68) (end 121.92 107.7468) (width 0.25) (layer "F.Cu") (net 1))
 (segment (start 124.8 106.1) (end 124.22 106.68) (width 0.25) (layer "F.Cu") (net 1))
 (segment (start 124.8 105.1) (end 124.8 106.1) (width 0.25) (layer "F.Cu") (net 1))
 (segment (start 121.92 107.7468) (end 121.92 112.77) (width 0.25) (layer "F.Cu") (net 1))
 (segment (start 131.1736 82.534) (end 129.8568 82.534) (width 0.25) (layer "F.Cu") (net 19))
 (segment (start 129.8568 82.534) (end 129.2352 83.1556) (width 0.25) (layer "F.Cu") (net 19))
 (segment (start 129.1336 84.2772) (end 129.2352 84.1756) (width 0.25) (layer "F.Cu") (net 12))
 (segment (start 128.27 84.2772) (end 129.1336 84.2772) (width 0.25) (layer "F.Cu") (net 12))
 (segment (start 128.3716 85.654) (end 128.3716 84.3788) (width 0.25) (layer "F.Cu") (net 12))
 (segment (start 128.3716 84.3788) (end 128.27 84.2772) (width 0.25) (layer "F.Cu") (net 12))
 (segment (start 129.2352 88.1648) (end 129.2 88.2) (width 0.25) (layer "F.Cu") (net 12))
 (segment (start 126.873 84.2772) (end 128.27 84.2772) (width 0.25) (layer "F.Cu") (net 12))
 (segment (start 129.2352 84.1756) (end 129.2352 88.1648) (width 0.25) (layer "F.Cu") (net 12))
 (segment (start 125.6 91.45) (end 127.7 91.45) (width 0.25) (layer "F.Cu") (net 2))
 (segment (start 123.7 105.1) (end 116.94 105.1) (width 0.25) (layer "F.Cu") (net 2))
 (segment (start 125.6 91.45) (end 125.6 101.95) (width 0.25) (layer "F.Cu") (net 2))
 (segment (start 137.675 103.775) (end 136.125 103.775) (width 0.25) (layer "F.Cu") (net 2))
 (segment (start 138 104.1) (end 137.675 103.775) (width 0.25) (layer "F.Cu") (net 2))
 (segment (start 123.7 105.1) (end 123.7 104.1) (width 0.25) (layer "F.Cu") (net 2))
 (segment (start 127.7 91.45) (end 129.8 91.45) (width 0.25) (layer "F.Cu") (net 2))
 (segment (start 120.18 84.68) (end 116.84 84.68) (width 0.25) (layer "F.Cu") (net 2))
 (segment (start 142.24 105.1) (end 142.24 105.08) (width 0.25) (layer "F.Cu") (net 2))
 (segment (start 123.5 97.75) (end 123.5 99.85) (width 0.25) (layer "F.Cu") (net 2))
 (segment (start 123.5 101.95) (end 123.5 99.85) (width 0.25) (layer "F.Cu") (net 2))
 (segment (start 138.2 95.65) (end 138.2 97.75) (width 0.25) (layer "F.Cu") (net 2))
 (segment (start 128.1 89.2) (end 128.425 89.525) (width 0.25) (layer "F.Cu") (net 2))
 (segment (start 138.2 101.95) (end 123.5 101.95) (width 0.25) (layer "F.Cu") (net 2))
 (segment (start 128.1 89.2) (end 127.775 89.525) (width 0.25) (layer "F.Cu") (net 2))
 (segment (start 123.7 104.1) (end 124.025 103.775) (width 0.25) (layer "F.Cu") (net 2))
 (segment (start 128.3716 86.614) (end 128.3716 87.9284) (width 0.25) (layer "F.Cu") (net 2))
 (segment (start 134 91.45) (end 136.1 91.45) (width 0.25) (layer "F.Cu") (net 2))
 (segment (start 135.8 105.1) (end 135.8 104.1) (width 0.25) (layer "F.Cu") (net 2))
 (segment (start 127.775 89.525) (end 124.025 89.525) (width 0.25) (layer "F.Cu") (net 2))
 (segment (start 127.7 91.45) (end 127.7 101.95) (width 0.25) (layer "F.Cu") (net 2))
 (segment (start 144.84 105.02) (end 144.84 102.48) (width 0.25) (layer "F.Cu") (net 2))
 (segment (start 144.76 105.1) (end 144.84 105.02) (width 0.25) (layer "F.Cu") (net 2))
 (segment (start 138.2 99.85) (end 138.2 101.95) (width 0.25) (layer "F.Cu") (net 2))
 (segment (start 131.9 91.45) (end 131.9 101.95) (width 0.25) (layer "F.Cu") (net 2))
 (segment (start 123.5 95.65) (end 138.2 95.65) (width 0.25) (layer "F.Cu") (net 2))
 (segment (start 128.425 89.525) (end 133.275 89.525) (width 0.25) (layer "F.Cu") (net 2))
 (segment (start 129.8 91.45) (end 129.8 101.95) (width 0.25) (layer "F.Cu") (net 2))
 (segment (start 138.2 97.75) (end 123.5 97.75) (width 0.25) (layer "F.Cu") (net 2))
 (segment (start 124.025 89.525) (end 123.7 89.2) (width 0.25) (layer "F.Cu") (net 2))
 (segment (start 121.92 88.9) (end 123 88.9) (width 0.25) (layer "F.Cu") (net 2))
 (segment (start 124.326 80.534) (end 120.18 84.68) (width 0.25) (layer "F.Cu") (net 2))
 (segment (start 125.575 103.775) (end 125.9 104.1) (width 0.25) (layer "F.Cu") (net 2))
 (segment (start 123.5 88.4) (end 123.7 88.2) (width 0.25) (layer "F.Cu") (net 2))
 (segment (start 123.5 99.85) (end 138.2 99.85) (width 0.25) (layer "F.Cu") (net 2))
 (segment (start 138 105.1) (end 138 104.1) (width 0.25) (layer "F.Cu") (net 2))
 (segment (start 123.5 91.45) (end 123.5 93.55) (width 0.25) (layer "F.Cu") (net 2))
 (segment (start 116.94 105.1) (end 116.84 105) (width 0.25) (layer "F.Cu") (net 2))
 (segment (start 119.85 96.6) (end 120.85 96.6) (width 0.25) (layer "F.Cu") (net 2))
 (segment (start 128.3716 87.9284) (end 128.1 88.2) (width 0.25) (layer "F.Cu") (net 2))
 (segment (start 123.5 91.45) (end 123.5 88.4) (width 0.25) (layer "F.Cu") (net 2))
 (segment (start 136.1 91.45) (end 136.1 101.95) (width 0.25) (layer "F.Cu") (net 2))
 (segment (start 138.2 91.45) (end 138.2 93.55) (width 0.25) (layer "F.Cu") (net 2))
 (segment (start 131.9 91.45) (end 134 91.45) (width 0.25) (layer "F.Cu") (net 2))
 (segment (start 138.2 91.45) (end 138.2 101.95) (width 0.25) (layer "F.Cu") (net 2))
 (segment (start 123.5 91.45) (end 125.6 91.45) (width 0.25) (layer "F.Cu") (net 2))
 (segment (start 133.275 89.525) (end 133.6 89.2) (width 0.25) (layer "F.Cu") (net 2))
 (segment (start 133.6 89.2) (end 133.6 88.2) (width 0.25) (layer "F.Cu") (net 2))
 (segment (start 131.0212 80.534) (end 124.326 80.534) (width 0.25) (layer "F.Cu") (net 2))
 (segment (start 136.1 91.45) (end 138.2 91.45) (width 0.25) (layer "F.Cu") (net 2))
 (segment (start 123 88.9) (end 123.7 88.2) (width 0.25) (layer "F.Cu") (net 2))
 (segment (start 138 105.1) (end 142.24 105.1) (width 0.25) (layer "F.Cu") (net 2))
 (segment (start 128.1 88.2) (end 128.1 89.2) (width 0.25) (layer "F.Cu") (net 2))
 (segment (start 134 91.45) (end 134 101.95) (width 0.25) (layer "F.Cu") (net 2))
 (segment (start 129.8 91.45) (end 131.9 91.45) (width 0.25) (layer "F.Cu") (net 2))
 (segment (start 121.92 95.53) (end 121.92 88.9) (width 0.25) (layer "F.Cu") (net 2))
 (segment (start 142.24 105.1) (end 144.76 105.1) (width 0.25) (layer "F.Cu") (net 2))
 (segment (start 123.5 93.55) (end 123.5 95.65) (width 0.25) (layer "F.Cu") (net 2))
 (segment (start 120.85 96.6) (end 121.92 95.53) (width 0.25) (layer "F.Cu") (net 2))
 (segment (start 125.9 104.1) (end 125.9 105.1) (width 0.25) (layer "F.Cu") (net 2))
 (segment (start 123.7 89.2) (end 123.7 88.2) (width 0.25) (layer "F.Cu") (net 2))
 (segment (start 136.125 103.775) (end 135.8 104.1) (width 0.25) (layer "F.Cu") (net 2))
 (segment (start 123.7 88.2) (end 120.18 84.68) (width 0.25) (layer "F.Cu") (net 2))
 (segment (start 124.025 103.775) (end 125.575 103.775) (width 0.25) (layer "F.Cu") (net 2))
 (segment (start 123.5 95.65) (end 123.5 97.75) (width 0.25) (layer "F.Cu") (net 2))
 (segment (start 138.2 93.55) (end 123.5 93.55) (width 0.25) (layer "F.Cu") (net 2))
 (segment (start 132.5372 86.7156) (end 131.4196 86.7156) (width 0.25) (layer "F.Cu") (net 11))
 (segment (start 144.84 84.7) (end 144.84 82.1344) (width 0.25) (layer "F.Cu") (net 11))
 (segment (start 124.317801 85.2932) (end 124.3838 85.227201) (width 0.25) (layer "F.Cu") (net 11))
 (segment (start 131.4 86.7352) (end 131.4 88.2) (width 0.25) (layer "F.Cu") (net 11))
 (segment (start 144.84 84.7) (end 146.0844 84.7) (width 0.25) (layer "F.Cu") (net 11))
 (segment (start 131.4196 86.7156) (end 131.4 86.7352) (width 0.25) (layer "F.Cu") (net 11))
 (segment (start 132.5372 88.1628) (end 132.5 88.2) (width 0.25) (layer "F.Cu") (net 11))
 (segment (start 146.0844 84.7) (end 146.4564 84.328) (width 0.25) (layer "F.Cu") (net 11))
 (segment (start 122.7836 85.2932) (end 124.317801 85.2932) (width 0.25) (layer "F.Cu") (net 11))
 (segment (start 132.5372 86.7156) (end 132.5372 88.1628) (width 0.25) (layer "F.Cu") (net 11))
 (segment (start 146.4564 84.328) (end 146.4564 78.1304) (width 0.25) (layer "F.Cu") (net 11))
 (segment (start 144.84 82.1344) (end 144.8816 82.0928) (width 0.25) (layer "F.Cu") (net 11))
 (via (at 144.8816 82.0928) (size 0.8) (drill 0.4) (layers "F.Cu" "B.Cu") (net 11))
 (via (at 122.7836 85.2932) (size 0.8) (drill 0.4) (layers "F.Cu" "B.Cu") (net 11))
 (via (at 146.4564 78.1304) (size 0.8) (drill 0.4) (layers "F.Cu" "B.Cu") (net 11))
 (via (at 132.5372 86.7156) (size 0.8) (drill 0.4) (layers "F.Cu" "B.Cu") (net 11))
 (segment (start 125.0696 78.1304) (end 121.7168 81.4832) (width 0.25) (layer "B.Cu") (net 11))
 (segment (start 121.7168 85.1408) (end 121.666 85.1916) (width 0.25) (layer "B.Cu") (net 11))
 (segment (start 121.7168 81.4832) (end 121.7168 85.1408) (width 0.25) (layer "B.Cu") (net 11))
 (segment (start 121.666 85.1916) (end 122.682 85.1916) (width 0.25) (layer "B.Cu") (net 11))
 (segment (start 137.16 82.0928) (end 132.5372 86.7156) (width 0.25) (layer "B.Cu") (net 11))
 (segment (start 122.682 85.1916) (end 122.7836 85.2932) (width 0.25) (layer "B.Cu") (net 11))
 (segment (start 146.4564 78.1304) (end 125.0696 78.1304) (width 0.25) (layer "B.Cu") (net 11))
 (segment (start 144.8816 82.0928) (end 137.16 82.0928) (width 0.25) (layer "B.Cu") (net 11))
 (segment (start 130.3 105.1) (end 130.3 103.38) (width 0.25) (layer "F.Cu") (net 3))
 (segment (start 130.3 103.38) (end 130.3528 103.3272) (width 0.25) (layer "F.Cu") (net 3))
 (via (at 130.3528 103.3272) (size 0.8) (drill 0.4) (layers "F.Cu" "B.Cu") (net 3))
 (segment (start 117.7072 103.3272) (end 116.84 102.46) (width 0.25) (layer "B.Cu") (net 3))
 (segment (start 130.3528 103.3272) (end 117.7072 103.3272) (width 0.25) (layer "B.Cu") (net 3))
 (segment (start 119.85 102.1) (end 119.02 102.1) (width 0.25) (layer "F.Cu") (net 18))
 (segment (start 119.02 102.1) (end 116.84 99.92) (width 0.25) (layer "F.Cu") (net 18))
 (segment (start 118.85 99.9) (end 116.84 97.89) (width 0.25) (layer "F.Cu") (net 17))
 (segment (start 119.85 99.9) (end 118.85 99.9) (width 0.25) (layer "F.Cu") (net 17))
 (segment (start 116.84 97.89) (end 116.84 97.38) (width 0.25) (layer "F.Cu") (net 17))
 (segment (start 118.015 96.015) (end 116.84 94.84) (width 0.25) (layer "F.Cu") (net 16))
 (segment (start 118.015 97.965) (end 118.015 96.015) (width 0.25) (layer "F.Cu") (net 16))
 (segment (start 119.85 98.8) (end 118.85 98.8) (width 0.25) (layer "F.Cu") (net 16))
 (segment (start 118.85 98.8) (end 118.015 97.965) (width 0.25) (layer "F.Cu") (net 16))
 (segment (start 119.85 97.7) (end 118.85 97.7) (width 0.25) (layer "F.Cu") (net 15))
 (segment (start 118.85 97.7) (end 118.465 97.315) (width 0.25) (layer "F.Cu") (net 15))
 (segment (start 118.465 93.925) (end 116.84 92.3) (width 0.25) (layer "F.Cu") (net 15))
 (segment (start 118.465 97.315) (end 118.465 93.925) (width 0.25) (layer "F.Cu") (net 15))
 (segment (start 119.85 91.1) (end 118.18 91.1) (width 0.25) (layer "F.Cu") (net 14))
 (segment (start 118.18 91.1) (end 116.84 89.76) (width 0.25) (layer "F.Cu") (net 14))
 (segment (start 119.85 90) (end 117.07 87.22) (width 0.25) (layer "F.Cu") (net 13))
 (segment (start 117.07 87.22) (end 116.84 87.22) (width 0.25) (layer "F.Cu") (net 13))
 (segment (start 141.85 90) (end 144.61 87.24) (width 0.25) (layer "F.Cu") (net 10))
 (segment (start 144.61 87.24) (end 144.84 87.24) (width 0.25) (layer "F.Cu") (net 10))
 (segment (start 143.52 91.1) (end 144.84 89.78) (width 0.25) (layer "F.Cu") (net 9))
 (segment (start 141.85 91.1) (end 143.52 91.1) (width 0.25) (layer "F.Cu") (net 9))
 (segment (start 141.85 97.7) (end 140.85 97.7) (width 0.25) (layer "F.Cu") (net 8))
 (segment (start 143.215 99.535) (end 143.215 96.485) (width 0.25) (layer "F.Cu") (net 7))
 (segment (start 143.215 96.485) (end 144.84 94.86) (width 0.25) (layer "F.Cu") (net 7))
 (segment (start 142.85 99.9) (end 143.215 99.535) (width 0.25) (layer "F.Cu") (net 7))
 (segment (start 141.85 99.9) (end 142.85 99.9) (width 0.25) (layer "F.Cu") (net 7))
 (segment (start 141.85 101) (end 143.091701 101) (width 0.25) (layer "F.Cu") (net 6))
 (segment (start 143.091701 101) (end 143.665 100.426701) (width 0.25) (layer "F.Cu") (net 6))
 (segment (start 143.665 100.426701) (end 143.665 98.575) (width 0.25) (layer "F.Cu") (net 6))
 (segment (start 143.665 98.575) (end 144.84 97.4) (width 0.25) (layer "F.Cu") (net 6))
 (segment (start 142.68 102.1) (end 144.84 99.94) (width 0.25) (layer "F.Cu") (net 5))
 (segment (start 141.85 102.1) (end 142.68 102.1) (width 0.25) (layer "F.Cu") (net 5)))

